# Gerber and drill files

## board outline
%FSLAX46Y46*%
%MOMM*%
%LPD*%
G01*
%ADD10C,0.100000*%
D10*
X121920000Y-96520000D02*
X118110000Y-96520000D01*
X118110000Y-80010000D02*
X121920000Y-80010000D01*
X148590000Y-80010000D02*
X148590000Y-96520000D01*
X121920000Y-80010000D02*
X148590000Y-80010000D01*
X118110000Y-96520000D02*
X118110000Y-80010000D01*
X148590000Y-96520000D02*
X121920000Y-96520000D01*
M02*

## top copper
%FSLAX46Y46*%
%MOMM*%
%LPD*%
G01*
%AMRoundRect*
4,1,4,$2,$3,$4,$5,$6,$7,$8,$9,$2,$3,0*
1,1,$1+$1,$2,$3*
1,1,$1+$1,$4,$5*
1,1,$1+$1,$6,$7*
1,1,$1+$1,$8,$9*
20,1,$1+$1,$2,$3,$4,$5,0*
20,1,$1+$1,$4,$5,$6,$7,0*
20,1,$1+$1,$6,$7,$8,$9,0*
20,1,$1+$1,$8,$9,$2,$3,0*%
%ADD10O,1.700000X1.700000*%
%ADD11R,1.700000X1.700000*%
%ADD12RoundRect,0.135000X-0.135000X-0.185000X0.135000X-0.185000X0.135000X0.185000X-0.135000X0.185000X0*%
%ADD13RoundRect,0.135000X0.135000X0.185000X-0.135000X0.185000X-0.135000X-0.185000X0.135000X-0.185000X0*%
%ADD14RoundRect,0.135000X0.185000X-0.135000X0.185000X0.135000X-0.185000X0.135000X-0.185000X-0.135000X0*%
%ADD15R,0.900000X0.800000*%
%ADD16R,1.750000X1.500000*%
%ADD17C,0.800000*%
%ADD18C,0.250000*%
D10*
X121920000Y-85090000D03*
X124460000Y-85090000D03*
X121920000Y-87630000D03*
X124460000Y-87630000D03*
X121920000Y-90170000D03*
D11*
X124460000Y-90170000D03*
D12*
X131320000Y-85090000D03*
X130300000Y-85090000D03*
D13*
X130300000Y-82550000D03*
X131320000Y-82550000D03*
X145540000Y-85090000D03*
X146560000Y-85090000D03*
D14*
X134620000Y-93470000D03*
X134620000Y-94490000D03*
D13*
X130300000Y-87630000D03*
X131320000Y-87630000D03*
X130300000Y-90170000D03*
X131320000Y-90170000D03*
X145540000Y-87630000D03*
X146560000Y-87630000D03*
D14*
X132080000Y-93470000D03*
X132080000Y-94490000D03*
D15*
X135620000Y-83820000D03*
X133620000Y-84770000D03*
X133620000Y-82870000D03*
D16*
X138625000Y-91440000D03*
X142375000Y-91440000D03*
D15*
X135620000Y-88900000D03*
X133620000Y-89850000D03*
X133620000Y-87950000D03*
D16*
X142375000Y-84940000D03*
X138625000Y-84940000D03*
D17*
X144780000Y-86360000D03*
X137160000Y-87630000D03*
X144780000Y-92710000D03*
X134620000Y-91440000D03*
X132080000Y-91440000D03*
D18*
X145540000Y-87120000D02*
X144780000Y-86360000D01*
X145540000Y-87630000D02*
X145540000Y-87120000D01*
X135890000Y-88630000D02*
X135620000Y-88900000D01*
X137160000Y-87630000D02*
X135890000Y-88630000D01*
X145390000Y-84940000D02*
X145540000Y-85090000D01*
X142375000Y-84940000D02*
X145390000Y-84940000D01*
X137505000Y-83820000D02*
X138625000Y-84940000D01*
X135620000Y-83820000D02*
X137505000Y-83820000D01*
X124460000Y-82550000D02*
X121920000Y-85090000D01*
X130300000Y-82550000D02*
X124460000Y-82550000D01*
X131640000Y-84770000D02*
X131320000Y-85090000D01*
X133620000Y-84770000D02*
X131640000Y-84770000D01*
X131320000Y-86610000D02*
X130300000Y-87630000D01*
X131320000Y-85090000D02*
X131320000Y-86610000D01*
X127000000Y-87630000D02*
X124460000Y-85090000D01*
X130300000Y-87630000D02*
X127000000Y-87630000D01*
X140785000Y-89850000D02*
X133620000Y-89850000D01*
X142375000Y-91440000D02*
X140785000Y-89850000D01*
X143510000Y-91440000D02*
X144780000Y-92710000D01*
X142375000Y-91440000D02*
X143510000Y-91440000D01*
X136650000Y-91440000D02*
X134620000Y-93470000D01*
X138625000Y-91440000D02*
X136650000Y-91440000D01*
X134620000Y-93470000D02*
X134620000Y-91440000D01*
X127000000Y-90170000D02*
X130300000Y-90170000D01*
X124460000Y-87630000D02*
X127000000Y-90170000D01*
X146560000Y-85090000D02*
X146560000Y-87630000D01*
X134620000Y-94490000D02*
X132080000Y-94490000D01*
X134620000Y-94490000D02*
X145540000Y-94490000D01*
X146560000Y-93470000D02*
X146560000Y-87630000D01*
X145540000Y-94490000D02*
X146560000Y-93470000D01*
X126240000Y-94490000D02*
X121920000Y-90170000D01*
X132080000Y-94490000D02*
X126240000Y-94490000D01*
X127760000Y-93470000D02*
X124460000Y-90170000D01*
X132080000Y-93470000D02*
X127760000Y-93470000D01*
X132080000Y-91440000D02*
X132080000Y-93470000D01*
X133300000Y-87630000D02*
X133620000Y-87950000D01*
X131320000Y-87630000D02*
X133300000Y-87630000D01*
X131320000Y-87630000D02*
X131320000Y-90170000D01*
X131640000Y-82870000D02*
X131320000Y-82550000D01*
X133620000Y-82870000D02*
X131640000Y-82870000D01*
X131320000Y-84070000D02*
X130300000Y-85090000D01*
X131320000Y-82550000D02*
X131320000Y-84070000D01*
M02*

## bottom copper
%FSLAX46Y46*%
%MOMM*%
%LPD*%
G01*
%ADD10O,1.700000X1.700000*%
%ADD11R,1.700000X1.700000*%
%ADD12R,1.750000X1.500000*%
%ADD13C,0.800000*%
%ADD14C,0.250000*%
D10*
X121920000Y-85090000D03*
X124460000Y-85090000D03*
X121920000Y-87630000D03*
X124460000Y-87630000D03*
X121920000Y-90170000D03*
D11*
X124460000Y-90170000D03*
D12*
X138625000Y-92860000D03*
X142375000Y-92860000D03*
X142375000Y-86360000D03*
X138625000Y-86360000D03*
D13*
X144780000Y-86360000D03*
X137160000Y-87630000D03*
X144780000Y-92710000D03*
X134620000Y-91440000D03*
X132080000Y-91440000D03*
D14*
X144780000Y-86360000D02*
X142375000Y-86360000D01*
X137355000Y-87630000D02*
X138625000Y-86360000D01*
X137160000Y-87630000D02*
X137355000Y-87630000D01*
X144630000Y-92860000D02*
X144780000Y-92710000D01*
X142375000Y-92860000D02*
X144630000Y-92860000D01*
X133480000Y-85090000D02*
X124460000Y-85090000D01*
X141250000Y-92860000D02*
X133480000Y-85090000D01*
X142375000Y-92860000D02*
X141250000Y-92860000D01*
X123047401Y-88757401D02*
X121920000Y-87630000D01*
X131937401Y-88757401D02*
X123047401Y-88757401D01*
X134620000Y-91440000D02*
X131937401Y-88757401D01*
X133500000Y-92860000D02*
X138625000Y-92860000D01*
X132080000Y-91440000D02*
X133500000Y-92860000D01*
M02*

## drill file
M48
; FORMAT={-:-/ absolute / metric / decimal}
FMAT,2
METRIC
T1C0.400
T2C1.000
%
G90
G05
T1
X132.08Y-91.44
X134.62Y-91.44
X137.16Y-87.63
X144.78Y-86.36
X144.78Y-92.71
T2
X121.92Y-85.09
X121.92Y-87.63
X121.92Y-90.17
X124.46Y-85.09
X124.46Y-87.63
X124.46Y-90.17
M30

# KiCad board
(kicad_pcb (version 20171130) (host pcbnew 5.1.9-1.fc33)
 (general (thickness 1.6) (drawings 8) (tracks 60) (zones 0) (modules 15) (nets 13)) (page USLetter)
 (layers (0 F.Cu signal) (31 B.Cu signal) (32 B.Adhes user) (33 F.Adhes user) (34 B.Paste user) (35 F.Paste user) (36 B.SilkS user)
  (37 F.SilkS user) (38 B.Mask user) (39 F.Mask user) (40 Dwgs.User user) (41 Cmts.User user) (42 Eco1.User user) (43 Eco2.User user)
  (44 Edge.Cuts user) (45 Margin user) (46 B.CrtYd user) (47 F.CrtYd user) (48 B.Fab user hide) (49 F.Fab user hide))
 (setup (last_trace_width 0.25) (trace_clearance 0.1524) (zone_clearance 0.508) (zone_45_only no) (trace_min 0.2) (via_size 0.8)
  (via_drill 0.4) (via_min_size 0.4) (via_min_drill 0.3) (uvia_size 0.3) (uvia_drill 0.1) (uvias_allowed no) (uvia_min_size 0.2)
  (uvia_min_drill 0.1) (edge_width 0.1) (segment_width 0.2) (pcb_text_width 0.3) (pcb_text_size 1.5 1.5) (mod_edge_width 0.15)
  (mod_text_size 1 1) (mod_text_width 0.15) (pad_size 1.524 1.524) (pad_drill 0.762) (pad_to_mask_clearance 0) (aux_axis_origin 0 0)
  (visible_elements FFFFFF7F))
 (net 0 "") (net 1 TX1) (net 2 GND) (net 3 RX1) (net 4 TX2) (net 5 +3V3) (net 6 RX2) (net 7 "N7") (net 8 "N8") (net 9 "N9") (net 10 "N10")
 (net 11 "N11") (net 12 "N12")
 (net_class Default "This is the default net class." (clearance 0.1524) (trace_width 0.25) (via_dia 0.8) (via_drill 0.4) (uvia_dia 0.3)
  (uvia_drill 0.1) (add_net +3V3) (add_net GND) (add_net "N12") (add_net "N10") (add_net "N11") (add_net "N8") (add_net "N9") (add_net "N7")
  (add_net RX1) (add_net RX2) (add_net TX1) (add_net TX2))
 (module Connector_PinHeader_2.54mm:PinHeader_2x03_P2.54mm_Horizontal (layer F.Cu) (at 124.46 90.17 180)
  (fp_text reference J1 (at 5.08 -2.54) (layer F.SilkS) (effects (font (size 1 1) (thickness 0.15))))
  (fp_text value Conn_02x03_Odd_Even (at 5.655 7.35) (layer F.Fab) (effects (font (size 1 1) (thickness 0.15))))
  (pad 6 thru_hole oval (at 2.54 5.08 180) (size 1.7 1.7) (drill 1) (layers *.Cu *.Mask) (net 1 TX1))
  (pad 5 thru_hole oval (at 0 5.08 180) (size 1.7 1.7) (drill 1) (layers *.Cu *.Mask) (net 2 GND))
  (pad 4 thru_hole oval (at 2.54 2.54 180) (size 1.7 1.7) (drill 1) (layers *.Cu *.Mask) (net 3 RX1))
  (pad 3 thru_hole oval (at 0 2.54 180) (size 1.7 1.7) (drill 1) (layers *.Cu *.Mask) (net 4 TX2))
  (pad 2 thru_hole oval (at 2.54 0 180) (size 1.7 1.7) (drill 1) (layers *.Cu *.Mask) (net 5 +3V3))
  (pad 1 thru_hole rect (at 0 0 180) (size 1.7 1.7) (drill 1) (layers *.Cu *.Mask) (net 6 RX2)))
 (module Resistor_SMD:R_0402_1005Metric (layer F.Cu) (at 130.81 85.09)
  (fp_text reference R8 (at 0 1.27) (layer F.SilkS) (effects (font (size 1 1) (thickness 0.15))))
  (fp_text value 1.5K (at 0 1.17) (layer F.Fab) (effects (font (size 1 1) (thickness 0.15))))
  (pad 2 smd roundrect (at 0.51 0) (size 0.54 0.64) (layers F.Cu F.Paste F.Mask) (roundrect_rratio 0.25) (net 2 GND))
  (pad 1 smd roundrect (at -0.51 0) (size 0.54 0.64) (layers F.Cu F.Paste F.Mask) (roundrect_rratio 0.25) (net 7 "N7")))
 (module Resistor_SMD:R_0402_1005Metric (layer F.Cu) (at 130.81 82.55 180)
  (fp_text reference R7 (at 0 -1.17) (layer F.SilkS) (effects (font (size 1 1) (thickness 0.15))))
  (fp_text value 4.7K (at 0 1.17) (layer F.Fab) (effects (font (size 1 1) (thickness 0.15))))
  (pad 2 smd roundrect (at 0.51 0 180) (size 0.54 0.64) (layers F.Cu F.Paste F.Mask) (roundrect_rratio 0.25) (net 1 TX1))
  (pad 1 smd roundrect (at -0.51 0 180) (size 0.54 0.64) (layers F.Cu F.Paste F.Mask) (roundrect_rratio 0.25) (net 7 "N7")))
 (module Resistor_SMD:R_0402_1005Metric (layer F.Cu) (at 146.05 85.09 180)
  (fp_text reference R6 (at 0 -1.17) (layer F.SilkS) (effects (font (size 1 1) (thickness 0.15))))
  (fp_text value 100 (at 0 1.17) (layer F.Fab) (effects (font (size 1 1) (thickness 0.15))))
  (pad 2 smd roundrect (at 0.51 0 180) (size 0.54 0.64) (layers F.Cu F.Paste F.Mask) (roundrect_rratio 0.25) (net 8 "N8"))
  (pad 1 smd roundrect (at -0.51 0 180) (size 0.54 0.64) (layers F.Cu F.Paste F.Mask) (roundrect_rratio 0.25) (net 5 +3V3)))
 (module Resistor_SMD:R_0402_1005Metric (layer F.Cu) (at 134.62 93.98 90)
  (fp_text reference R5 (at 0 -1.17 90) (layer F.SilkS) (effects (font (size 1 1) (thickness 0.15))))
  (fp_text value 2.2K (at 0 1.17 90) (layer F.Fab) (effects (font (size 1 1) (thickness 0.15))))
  (pad 2 smd roundrect (at 0.51 0 90) (size 0.54 0.64) (layers F.Cu F.Paste F.Mask) (roundrect_rratio 0.25) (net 3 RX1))
  (pad 1 smd roundrect (at -0.51 0 90) (size 0.54 0.64) (layers F.Cu F.Paste F.Mask) (roundrect_rratio 0.25) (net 5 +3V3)))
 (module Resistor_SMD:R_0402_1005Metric (layer F.Cu) (at 130.81 87.63 180)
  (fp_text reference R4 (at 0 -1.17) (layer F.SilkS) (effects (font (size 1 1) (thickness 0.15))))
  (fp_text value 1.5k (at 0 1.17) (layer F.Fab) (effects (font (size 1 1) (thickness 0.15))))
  (pad 2 smd roundrect (at 0.51 0 180) (size 0.54 0.64) (layers F.Cu F.Paste F.Mask) (roundrect_rratio 0.25) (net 2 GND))
  (pad 1 smd roundrect (at -0.51 0 180) (size 0.54 0.64) (layers F.Cu F.Paste F.Mask) (roundrect_rratio 0.25) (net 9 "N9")))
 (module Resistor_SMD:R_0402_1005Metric (layer F.Cu) (at 130.81 90.17 180)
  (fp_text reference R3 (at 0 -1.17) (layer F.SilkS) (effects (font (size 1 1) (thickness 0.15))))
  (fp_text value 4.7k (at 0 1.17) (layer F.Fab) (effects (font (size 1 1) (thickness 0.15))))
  (pad 2 smd roundrect (at 0.51 0 180) (size 0.54 0.64) (layers F.Cu F.Paste F.Mask) (roundrect_rratio 0.25) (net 4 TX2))
  (pad 1 smd roundrect (at -0.51 0 180) (size 0.54 0.64) (layers F.Cu F.Paste F.Mask) (roundrect_rratio 0.25) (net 9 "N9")))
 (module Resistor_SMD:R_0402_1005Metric (layer F.Cu) (at 146.05 87.63 180)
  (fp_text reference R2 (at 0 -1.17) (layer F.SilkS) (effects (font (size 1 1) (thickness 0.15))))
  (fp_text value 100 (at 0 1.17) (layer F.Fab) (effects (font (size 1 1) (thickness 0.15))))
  (pad 2 smd roundrect (at 0.51 0 180) (size 0.54 0.64) (layers F.Cu F.Paste F.Mask) (roundrect_rratio 0.25) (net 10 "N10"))
  (pad 1 smd roundrect (at -0.51 0 180) (size 0.54 0.64) (layers F.Cu F.Paste F.Mask) (roundrect_rratio 0.25) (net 5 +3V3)))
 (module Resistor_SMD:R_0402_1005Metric (layer F.Cu) (at 132.08 93.98 90)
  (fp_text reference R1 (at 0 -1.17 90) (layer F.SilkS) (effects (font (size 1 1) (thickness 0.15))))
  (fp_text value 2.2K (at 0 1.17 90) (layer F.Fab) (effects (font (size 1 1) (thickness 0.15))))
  (pad 2 smd roundrect (at 0.51 0 90) (size 0.54 0.64) (layers F.Cu F.Paste F.Mask) (roundrect_rratio 0.25) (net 6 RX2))
  (pad 1 smd roundrect (at -0.51 0 90) (size 0.54 0.64) (layers F.Cu F.Paste F.Mask) (roundrect_rratio 0.25) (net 5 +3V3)))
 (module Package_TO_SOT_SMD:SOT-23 (layer F.Cu) (at 134.62 83.82)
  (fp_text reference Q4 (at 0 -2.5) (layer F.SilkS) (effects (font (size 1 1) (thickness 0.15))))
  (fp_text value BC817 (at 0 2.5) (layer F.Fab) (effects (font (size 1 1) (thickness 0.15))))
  (pad 3 smd rect (at 1 0) (size 0.9 0.8) (layers F.Cu F.Paste F.Mask) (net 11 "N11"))
  (pad 2 smd rect (at -1 0.95) (size 0.9 0.8) (layers F.Cu F.Paste F.Mask) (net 2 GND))
  (pad 1 smd rect (at -1 -0.95) (size 0.9 0.8) (layers F.Cu F.Paste F.Mask) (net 7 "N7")))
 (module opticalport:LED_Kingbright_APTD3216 (layer F.Cu) (at 140.5 91.44 180)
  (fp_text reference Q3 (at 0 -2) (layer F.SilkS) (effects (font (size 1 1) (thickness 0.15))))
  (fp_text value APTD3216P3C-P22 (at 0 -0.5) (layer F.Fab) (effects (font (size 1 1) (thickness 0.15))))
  (pad 2 smd rect (at 1.875 0 180) (size 1.75 1.5) (layers F.Cu F.Paste F.Mask) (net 3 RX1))
  (pad 1 smd rect (at -1.875 0 180) (size 1.75 1.5) (layers F.Cu F.Paste F.Mask) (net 2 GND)))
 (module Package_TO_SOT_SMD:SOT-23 (layer F.Cu) (at 134.62 88.9)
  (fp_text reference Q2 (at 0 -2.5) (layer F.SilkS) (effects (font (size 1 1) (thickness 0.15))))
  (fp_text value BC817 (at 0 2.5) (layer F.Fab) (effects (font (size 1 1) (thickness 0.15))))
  (pad 3 smd rect (at 1 0) (size 0.9 0.8) (layers F.Cu F.Paste F.Mask) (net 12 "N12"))
  (pad 2 smd rect (at -1 0.95) (size 0.9 0.8) (layers F.Cu F.Paste F.Mask) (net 2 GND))
  (pad 1 smd rect (at -1 -0.95) (size 0.9 0.8) (layers F.Cu F.Paste F.Mask) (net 9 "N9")))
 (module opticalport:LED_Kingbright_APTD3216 (layer B.Cu) (at 140.5 92.86 180)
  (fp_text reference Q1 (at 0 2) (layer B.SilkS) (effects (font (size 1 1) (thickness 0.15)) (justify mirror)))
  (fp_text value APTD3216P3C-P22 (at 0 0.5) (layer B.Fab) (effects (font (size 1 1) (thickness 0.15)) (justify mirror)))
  (pad 2 smd rect (at 1.875 0 180) (size 1.75 1.5) (layers B.Cu B.Paste B.Mask) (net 6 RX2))
  (pad 1 smd rect (at -1.875 0 180) (size 1.75 1.5) (layers B.Cu B.Paste B.Mask) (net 2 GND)))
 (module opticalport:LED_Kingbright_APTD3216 (layer F.Cu) (at 140.5 84.94)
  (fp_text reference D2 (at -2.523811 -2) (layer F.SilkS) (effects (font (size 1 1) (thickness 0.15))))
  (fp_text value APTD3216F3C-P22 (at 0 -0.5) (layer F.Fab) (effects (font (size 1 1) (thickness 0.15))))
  (pad 2 smd rect (at 1.875 0) (size 1.75 1.5) (layers F.Cu F.Paste F.Mask) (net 8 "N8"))
  (pad 1 smd rect (at -1.875 0) (size 1.75 1.5) (layers F.Cu F.Paste F.Mask) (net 11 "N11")))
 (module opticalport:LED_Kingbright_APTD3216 (layer B.Cu) (at 140.5 86.36)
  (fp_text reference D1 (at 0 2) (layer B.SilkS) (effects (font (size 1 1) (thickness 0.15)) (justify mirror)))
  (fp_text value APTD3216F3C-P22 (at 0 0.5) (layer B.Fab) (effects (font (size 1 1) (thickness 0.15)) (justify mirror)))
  (pad 2 smd rect (at 1.875 0) (size 1.75 1.5) (layers B.Cu B.Paste B.Mask) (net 10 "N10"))
  (pad 1 smd rect (at -1.875 0) (size 1.75 1.5) (layers B.Cu B.Paste B.Mask) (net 12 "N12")))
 (gr_line (start 121.92 96.52) (end 118.11 96.52) (layer Edge.Cuts) (width 0.1))
 (gr_line (start 118.11 80.01) (end 121.92 80.01) (layer Edge.Cuts) (width 0.1))
 (gr_line (start 148.59 80.01) (end 148.59 96.52) (layer Edge.Cuts) (width 0.1))
 (gr_line (start 121.92 80.01) (end 148.59 80.01) (layer Edge.Cuts) (width 0.1))
 (gr_line (start 118.11 96.52) (end 118.11 80.01) (layer Edge.Cuts) (width 0.1))
 (gr_line (start 148.59 96.52) (end 121.92 96.52) (layer Edge.Cuts) (width 0.1))
 (via (at 144.78 86.36) (size 0.8) (drill 0.4) (layers F.Cu B.Cu) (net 10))
 (segment (start 145.54 87.12) (end 144.78 86.36) (width 0.25) (layer F.Cu) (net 10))
 (segment (start 145.54 87.63) (end 145.54 87.12) (width 0.25) (layer F.Cu) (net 10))
 (segment (start 144.78 86.36) (end 142.375 86.36) (width 0.25) (layer B.Cu) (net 10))
 (segment (start 135.89 88.63) (end 135.62 88.9) (width 0.25) (layer F.Cu) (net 12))
 (segment (start 137.16 87.63) (end 135.89 88.63) (width 0.25) (layer F.Cu) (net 12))
 (via (at 137.16 87.63) (size 0.8) (drill 0.4) (layers F.Cu B.Cu) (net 12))
 (segment (start 137.355 87.63) (end 138.625 86.36) (width 0.25) (layer B.Cu) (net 12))
 (segment (start 137.16 87.63) (end 137.355 87.63) (width 0.25) (layer B.Cu) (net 12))
 (segment (start 145.39 84.94) (end 145.54 85.09) (width 0.25) (layer F.Cu) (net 8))
 (segment (start 142.375 84.94) (end 145.39 84.94) (width 0.25) (layer F.Cu) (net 8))
 (segment (start 137.505 83.82) (end 138.625 84.94) (width 0.25) (layer F.Cu) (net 11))
 (segment (start 135.62 83.82) (end 137.505 83.82) (width 0.25) (layer F.Cu) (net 11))
 (segment (start 124.46 82.55) (end 121.92 85.09) (width 0.25) (layer F.Cu) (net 1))
 (segment (start 130.3 82.55) (end 124.46 82.55) (width 0.25) (layer F.Cu) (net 1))
 (segment (start 131.64 84.77) (end 131.32 85.09) (width 0.25) (layer F.Cu) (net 2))
 (segment (start 133.62 84.77) (end 131.64 84.77) (width 0.25) (layer F.Cu) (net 2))
 (segment (start 131.32 86.61) (end 130.3 87.63) (width 0.25) (layer F.Cu) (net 2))
 (segment (start 131.32 85.09) (end 131.32 86.61) (width 0.25) (layer F.Cu) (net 2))
 (segment (start 127 87.63) (end 124.46 85.09) (width 0.25) (layer F.Cu) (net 2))
 (segment (start 130.3 87.63) (end 127 87.63) (width 0.25) (layer F.Cu) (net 2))
 (segment (start 140.785 89.85) (end 133.62 89.85) (width 0.25) (layer F.Cu) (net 2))
 (segment (start 142.375 91.44) (end 140.785 89.85) (width 0.25) (layer F.Cu) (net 2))
 (via (at 144.78 92.71) (size 0.8) (drill 0.4) (layers F.Cu B.Cu) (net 2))
 (segment (start 143.51 91.44) (end 144.78 92.71) (width 0.25) (layer F.Cu) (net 2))
 (segment (start 142.375 91.44) (end 143.51 91.44) (width 0.25) (layer F.Cu) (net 2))
 (segment (start 144.63 92.86) (end 144.78 92.71) (width 0.25) (layer B.Cu) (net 2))
 (segment (start 142.375 92.86) (end 144.63 92.86) (width 0.25) (layer B.Cu) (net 2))
 (segment (start 133.48 85.09) (end 124.46 85.09) (width 0.25) (layer B.Cu) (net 2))
 (segment (start 141.25 92.86) (end 133.48 85.09) (width 0.25) (layer B.Cu) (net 2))
 (segment (start 142.375 92.86) (end 141.25 92.86) (width 0.25) (layer B.Cu) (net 2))
 (segment (start 136.65 91.44) (end 134.62 93.47) (width 0.25) (layer F.Cu) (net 3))
 (segment (start 138.625 91.44) (end 136.65 91.44) (width 0.25) (layer F.Cu) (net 3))
 (via (at 134.62 91.44) (size 0.8) (drill 0.4) (layers F.Cu B.Cu) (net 3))
 (segment (start 134.62 93.47) (end 134.62 91.44) (width 0.25) (layer F.Cu) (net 3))
 (segment (start 123.047401 88.757401) (end 121.92 87.63) (width 0.25) (layer B.Cu) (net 3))
 (segment (start 131.937401 88.757401) (end 123.047401 88.757401) (width 0.25) (layer B.Cu) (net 3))
 (segment (start 134.62 91.44) (end 131.937401 88.757401) (width 0.25) (layer B.Cu) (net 3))
 (segment (start 127 90.17) (end 130.3 90.17) (width 0.25) (layer F.Cu) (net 4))
 (segment (start 124.46 87.63) (end 127 90.17) (width 0.25) (layer F.Cu) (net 4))
 (segment (start 146.56 85.09) (end 146.56 87.63) (width 0.25) (layer F.Cu) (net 5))
 (segment (start 134.62 94.49) (end 132.08 94.49) (width 0.25) (layer F.Cu) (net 5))
 (segment (start 134.62 94.49) (end 145.54 94.49) (width 0.25) (layer F.Cu) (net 5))
 (segment (start 146.56 93.47) (end 146.56 87.63) (width 0.25) (layer F.Cu) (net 5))
 (segment (start 145.54 94.49) (end 146.56 93.47) (width 0.25) (layer F.Cu) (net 5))
 (segment (start 126.24 94.49) (end 121.92 90.17) (width 0.25) (layer F.Cu) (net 5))
 (segment (start 132.08 94.49) (end 126.24 94.49) (width 0.25) (layer F.Cu) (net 5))
 (segment (start 127.76 93.47) (end 124.46 90.17) (width 0.25) (layer F.Cu) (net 6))
 (segment (start 132.08 93.47) (end 127.76 93.47) (width 0.25) (layer F.Cu) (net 6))
 (via (at 132.08 91.44) (size 0.8) (drill 0.4) (layers F.Cu B.Cu) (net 6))
 (segment (start 132.08 91.44) (end 132.08 93.47) (width 0.25) (layer F.Cu) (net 6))
 (segment (start 133.5 92.86) (end 138.625 92.86) (width 0.25) (layer B.Cu) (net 6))
 (segment (start 132.08 91.44) (end 133.5 92.86) (width 0.25) (layer B.Cu) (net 6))
 (segment (start 133.3 87.63) (end 133.62 87.95) (width 0.25) (layer F.Cu) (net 9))
 (segment (start 131.32 87.63) (end 133.3 87.63) (width 0.25) (layer F.Cu) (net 9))
 (segment (start 131.32 87.63) (end 131.32 90.17) (width 0.25) (layer F.Cu) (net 9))
 (segment (start 131.64 82.87) (end 131.32 82.55) (width 0.25) (layer F.Cu) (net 7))
 (segment (start 133.62 82.87) (end 131.64 82.87) (width 0.25) (layer F.Cu) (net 7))
 (segment (start 131.32 84.07) (end 130.3 85.09) (width 0.25) (layer F.Cu) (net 7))
 (segment (start 131.32 82.55) (end 131.32 84.07) (width 0.25) (layer F.Cu) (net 7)))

